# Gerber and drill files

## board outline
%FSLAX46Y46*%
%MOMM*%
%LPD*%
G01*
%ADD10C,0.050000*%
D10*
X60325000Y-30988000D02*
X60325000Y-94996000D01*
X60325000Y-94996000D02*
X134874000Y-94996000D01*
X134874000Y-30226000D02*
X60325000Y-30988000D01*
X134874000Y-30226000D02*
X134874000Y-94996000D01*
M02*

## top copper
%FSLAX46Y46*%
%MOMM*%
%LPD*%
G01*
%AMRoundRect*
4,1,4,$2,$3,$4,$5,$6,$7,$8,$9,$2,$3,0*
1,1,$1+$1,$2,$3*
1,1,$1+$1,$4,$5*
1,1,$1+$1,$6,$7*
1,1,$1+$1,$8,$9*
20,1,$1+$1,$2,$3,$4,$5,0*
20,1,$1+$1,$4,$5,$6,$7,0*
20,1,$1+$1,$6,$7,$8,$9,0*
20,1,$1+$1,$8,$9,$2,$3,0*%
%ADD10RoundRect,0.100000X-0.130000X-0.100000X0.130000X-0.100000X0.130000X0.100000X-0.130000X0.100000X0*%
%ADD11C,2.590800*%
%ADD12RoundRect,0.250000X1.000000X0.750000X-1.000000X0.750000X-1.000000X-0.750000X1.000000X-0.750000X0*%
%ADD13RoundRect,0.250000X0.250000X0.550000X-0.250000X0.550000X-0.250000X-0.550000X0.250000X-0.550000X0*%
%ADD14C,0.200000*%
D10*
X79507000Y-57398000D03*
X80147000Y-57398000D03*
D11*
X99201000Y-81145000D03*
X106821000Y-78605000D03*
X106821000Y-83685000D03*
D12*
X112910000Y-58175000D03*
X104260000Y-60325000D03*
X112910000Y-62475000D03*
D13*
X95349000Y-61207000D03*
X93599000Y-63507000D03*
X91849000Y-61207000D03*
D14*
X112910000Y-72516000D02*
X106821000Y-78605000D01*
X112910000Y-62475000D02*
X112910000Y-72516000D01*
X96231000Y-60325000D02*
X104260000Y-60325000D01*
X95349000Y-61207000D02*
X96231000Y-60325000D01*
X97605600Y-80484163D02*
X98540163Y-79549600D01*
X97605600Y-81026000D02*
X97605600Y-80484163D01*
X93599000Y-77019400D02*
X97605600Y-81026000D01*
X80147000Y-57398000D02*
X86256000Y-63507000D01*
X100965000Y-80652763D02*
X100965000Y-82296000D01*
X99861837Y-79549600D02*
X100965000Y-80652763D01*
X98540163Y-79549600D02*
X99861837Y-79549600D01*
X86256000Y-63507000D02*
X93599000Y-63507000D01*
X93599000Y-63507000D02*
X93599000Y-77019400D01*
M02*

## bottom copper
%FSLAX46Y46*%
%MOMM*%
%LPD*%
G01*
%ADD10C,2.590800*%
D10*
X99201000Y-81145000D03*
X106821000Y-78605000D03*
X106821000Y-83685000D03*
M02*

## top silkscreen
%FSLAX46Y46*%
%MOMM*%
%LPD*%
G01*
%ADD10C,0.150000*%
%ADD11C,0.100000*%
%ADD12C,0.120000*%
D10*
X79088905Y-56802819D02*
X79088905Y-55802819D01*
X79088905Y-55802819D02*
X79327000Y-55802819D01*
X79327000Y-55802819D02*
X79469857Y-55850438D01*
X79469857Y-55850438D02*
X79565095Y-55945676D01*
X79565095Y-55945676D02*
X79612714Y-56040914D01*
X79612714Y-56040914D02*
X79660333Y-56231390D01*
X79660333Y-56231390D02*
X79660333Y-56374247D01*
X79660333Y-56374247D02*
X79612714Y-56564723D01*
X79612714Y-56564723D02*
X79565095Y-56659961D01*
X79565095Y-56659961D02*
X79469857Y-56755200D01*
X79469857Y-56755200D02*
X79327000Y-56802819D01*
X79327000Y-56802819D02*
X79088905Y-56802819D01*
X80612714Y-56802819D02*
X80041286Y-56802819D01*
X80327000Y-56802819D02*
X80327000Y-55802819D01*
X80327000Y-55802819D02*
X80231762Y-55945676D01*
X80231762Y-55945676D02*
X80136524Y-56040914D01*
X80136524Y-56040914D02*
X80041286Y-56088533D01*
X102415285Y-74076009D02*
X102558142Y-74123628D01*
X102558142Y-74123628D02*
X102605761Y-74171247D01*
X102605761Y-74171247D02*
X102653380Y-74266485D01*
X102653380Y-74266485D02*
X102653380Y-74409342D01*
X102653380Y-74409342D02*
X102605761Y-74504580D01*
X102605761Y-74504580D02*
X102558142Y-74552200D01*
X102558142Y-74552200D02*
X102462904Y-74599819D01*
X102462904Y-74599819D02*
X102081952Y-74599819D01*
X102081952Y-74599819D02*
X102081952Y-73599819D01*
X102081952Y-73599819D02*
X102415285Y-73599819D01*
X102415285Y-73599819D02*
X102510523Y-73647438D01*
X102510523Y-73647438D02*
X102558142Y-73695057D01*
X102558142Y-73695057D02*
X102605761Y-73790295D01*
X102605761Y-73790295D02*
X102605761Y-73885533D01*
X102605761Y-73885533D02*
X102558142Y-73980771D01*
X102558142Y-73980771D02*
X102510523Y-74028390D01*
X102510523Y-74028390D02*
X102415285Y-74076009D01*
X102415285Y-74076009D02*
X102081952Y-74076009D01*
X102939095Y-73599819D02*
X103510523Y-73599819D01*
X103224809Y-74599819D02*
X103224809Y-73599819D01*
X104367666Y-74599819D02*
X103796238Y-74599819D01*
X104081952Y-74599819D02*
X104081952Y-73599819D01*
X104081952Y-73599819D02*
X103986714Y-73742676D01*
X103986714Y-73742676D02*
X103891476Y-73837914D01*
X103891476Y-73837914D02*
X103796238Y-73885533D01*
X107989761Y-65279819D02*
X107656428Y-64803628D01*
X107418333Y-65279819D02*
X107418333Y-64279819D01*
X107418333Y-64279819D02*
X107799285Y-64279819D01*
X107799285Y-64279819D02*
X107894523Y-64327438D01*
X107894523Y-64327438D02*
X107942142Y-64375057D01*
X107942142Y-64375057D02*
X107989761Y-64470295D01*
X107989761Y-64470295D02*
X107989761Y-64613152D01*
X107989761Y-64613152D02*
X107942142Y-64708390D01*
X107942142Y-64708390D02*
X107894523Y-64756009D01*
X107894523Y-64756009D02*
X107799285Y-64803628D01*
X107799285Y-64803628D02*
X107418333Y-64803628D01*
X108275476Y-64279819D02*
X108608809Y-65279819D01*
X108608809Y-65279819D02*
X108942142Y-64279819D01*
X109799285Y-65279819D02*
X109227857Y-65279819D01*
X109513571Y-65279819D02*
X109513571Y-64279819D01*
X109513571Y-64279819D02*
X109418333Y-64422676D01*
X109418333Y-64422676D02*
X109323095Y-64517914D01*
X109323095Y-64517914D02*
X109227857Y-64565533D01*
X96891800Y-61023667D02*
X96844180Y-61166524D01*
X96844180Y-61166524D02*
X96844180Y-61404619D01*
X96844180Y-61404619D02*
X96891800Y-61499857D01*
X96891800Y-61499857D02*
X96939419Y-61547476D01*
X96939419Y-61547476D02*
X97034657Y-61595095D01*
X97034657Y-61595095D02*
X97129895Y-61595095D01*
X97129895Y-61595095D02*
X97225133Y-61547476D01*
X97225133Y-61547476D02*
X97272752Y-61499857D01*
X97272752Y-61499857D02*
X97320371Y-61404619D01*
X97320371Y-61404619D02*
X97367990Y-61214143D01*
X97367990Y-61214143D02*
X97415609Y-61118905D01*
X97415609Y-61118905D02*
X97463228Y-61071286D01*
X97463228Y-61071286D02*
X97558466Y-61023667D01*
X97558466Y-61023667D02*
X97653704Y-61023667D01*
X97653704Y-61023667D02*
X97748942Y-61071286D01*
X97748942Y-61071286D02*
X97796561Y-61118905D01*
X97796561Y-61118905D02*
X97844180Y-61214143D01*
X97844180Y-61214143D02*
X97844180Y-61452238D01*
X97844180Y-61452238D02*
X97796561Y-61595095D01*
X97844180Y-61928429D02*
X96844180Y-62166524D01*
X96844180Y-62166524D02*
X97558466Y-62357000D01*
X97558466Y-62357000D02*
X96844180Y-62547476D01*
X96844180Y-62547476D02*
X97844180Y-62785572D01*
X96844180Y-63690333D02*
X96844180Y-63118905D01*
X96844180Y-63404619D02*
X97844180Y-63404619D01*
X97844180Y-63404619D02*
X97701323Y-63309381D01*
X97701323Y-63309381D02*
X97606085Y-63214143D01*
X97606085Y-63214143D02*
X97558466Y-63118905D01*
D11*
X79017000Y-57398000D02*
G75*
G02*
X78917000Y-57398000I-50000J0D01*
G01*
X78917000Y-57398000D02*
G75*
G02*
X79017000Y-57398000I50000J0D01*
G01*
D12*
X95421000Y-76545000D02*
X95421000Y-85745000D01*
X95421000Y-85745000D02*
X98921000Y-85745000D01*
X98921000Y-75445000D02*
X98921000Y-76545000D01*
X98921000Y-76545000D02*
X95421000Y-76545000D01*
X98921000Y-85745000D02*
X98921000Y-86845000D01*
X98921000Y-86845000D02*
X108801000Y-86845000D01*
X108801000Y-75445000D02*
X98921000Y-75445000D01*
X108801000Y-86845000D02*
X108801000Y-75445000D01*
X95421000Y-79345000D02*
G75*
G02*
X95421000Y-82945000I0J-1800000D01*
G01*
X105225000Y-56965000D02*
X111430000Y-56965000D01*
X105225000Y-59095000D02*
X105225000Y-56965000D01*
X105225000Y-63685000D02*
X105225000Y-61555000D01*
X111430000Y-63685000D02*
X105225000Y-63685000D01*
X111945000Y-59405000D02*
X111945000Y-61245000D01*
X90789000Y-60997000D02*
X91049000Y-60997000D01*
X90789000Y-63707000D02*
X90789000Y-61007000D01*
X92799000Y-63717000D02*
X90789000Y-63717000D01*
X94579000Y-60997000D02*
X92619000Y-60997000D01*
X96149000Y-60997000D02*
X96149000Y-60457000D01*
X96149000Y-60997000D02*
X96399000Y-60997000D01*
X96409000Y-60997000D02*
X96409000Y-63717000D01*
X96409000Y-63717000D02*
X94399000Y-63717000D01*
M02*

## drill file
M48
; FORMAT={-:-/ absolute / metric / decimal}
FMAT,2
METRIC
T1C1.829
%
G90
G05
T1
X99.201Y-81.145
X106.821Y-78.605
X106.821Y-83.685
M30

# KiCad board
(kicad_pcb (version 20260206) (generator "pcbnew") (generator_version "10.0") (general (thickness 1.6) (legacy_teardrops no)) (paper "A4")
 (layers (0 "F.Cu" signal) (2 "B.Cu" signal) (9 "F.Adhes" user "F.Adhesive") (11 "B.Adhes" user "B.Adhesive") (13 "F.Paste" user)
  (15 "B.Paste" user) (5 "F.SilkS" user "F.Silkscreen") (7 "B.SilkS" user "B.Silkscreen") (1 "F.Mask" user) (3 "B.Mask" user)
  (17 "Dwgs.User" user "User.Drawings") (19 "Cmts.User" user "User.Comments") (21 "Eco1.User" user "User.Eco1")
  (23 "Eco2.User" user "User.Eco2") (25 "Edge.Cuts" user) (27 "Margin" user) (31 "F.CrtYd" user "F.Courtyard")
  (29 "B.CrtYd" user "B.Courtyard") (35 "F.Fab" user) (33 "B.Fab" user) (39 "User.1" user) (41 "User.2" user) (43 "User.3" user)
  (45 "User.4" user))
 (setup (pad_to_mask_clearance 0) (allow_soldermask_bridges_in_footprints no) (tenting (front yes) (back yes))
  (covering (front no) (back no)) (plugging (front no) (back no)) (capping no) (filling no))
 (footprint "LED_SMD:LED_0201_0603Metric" (layer "F.Cu") (at 79.827 57.398)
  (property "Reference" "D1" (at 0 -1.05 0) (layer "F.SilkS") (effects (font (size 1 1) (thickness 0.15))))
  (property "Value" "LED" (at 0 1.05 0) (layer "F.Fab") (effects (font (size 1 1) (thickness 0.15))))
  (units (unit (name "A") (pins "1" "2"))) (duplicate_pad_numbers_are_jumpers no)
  (fp_circle (center -0.86 0) (end -0.81 0) (stroke (width 0.1) (type solid)) (fill no) (layer "F.SilkS"))
  (pad "" smd roundrect (at -0.345 0) (size 0.318 0.36) (layers "F.Paste") (roundrect_rratio 0.25))
  (pad "" smd roundrect (at 0.345 0) (size 0.318 0.36) (layers "F.Paste") (roundrect_rratio 0.25))
  (pad "1" smd roundrect (at -0.32 0) (size 0.46 0.4) (layers "F.Cu" "F.Mask") (roundrect_rratio 0.25) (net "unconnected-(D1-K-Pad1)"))
  (pad "2" smd roundrect (at 0.32 0) (size 0.46 0.4) (layers "F.Cu" "F.Mask") (roundrect_rratio 0.25) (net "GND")))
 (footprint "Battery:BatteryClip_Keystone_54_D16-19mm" (layer "F.Cu") (at 99.201 81.145)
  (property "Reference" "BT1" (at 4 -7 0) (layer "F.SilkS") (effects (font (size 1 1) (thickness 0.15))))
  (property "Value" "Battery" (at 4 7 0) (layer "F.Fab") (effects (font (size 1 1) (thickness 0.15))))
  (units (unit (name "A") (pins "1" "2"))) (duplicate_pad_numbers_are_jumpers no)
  (fp_line (start -3.78 -4.6) (end -3.78 4.6) (stroke (width 0.12) (type default)) (layer "F.SilkS"))
  (fp_line (start -3.78 4.6) (end -0.28 4.6) (stroke (width 0.12) (type default)) (layer "F.SilkS"))
  (fp_line (start -0.28 -5.7) (end -0.28 -4.6) (stroke (width 0.12) (type default)) (layer "F.SilkS"))
  (fp_line (start -0.28 -4.6) (end -3.78 -4.6) (stroke (width 0.12) (type default)) (layer "F.SilkS"))
  (fp_line (start -0.28 4.6) (end -0.28 5.7) (stroke (width 0.12) (type default)) (layer "F.SilkS"))
  (fp_line (start -0.28 5.7) (end 9.6 5.7) (stroke (width 0.12) (type default)) (layer "F.SilkS"))
  (fp_line (start 9.6 -5.7) (end -0.28 -5.7) (stroke (width 0.12) (type default)) (layer "F.SilkS"))
  (fp_line (start 9.6 5.7) (end 9.6 -5.7) (stroke (width 0.12) (type default)) (layer "F.SilkS"))
  (fp_arc (start -3.78 -1.8) (mid -1.98 0) (end -3.78 1.8) (stroke (width 0.12) (type default)) (layer "F.SilkS"))
  (pad "1" thru_hole circle (at 0 0 180) (size 2.5908 2.5908) (drill 1.8288) (layers "*.Cu" "*.Mask") (remove_unused_layers no) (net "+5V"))
  (pad "1" thru_hole circle (at 7.62 -2.54 180) (size 2.5908 2.5908) (drill 1.8288) (layers "*.Cu" "*.Mask") (remove_unused_layers no)
   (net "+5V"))
  (pad "1" thru_hole circle (at 7.62 2.54 180) (size 2.5908 2.5908) (drill 1.8288) (layers "*.Cu" "*.Mask") (remove_unused_layers no)
   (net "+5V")))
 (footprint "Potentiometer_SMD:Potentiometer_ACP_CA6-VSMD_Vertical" (layer "F.Cu") (at 108.585 60.325 180)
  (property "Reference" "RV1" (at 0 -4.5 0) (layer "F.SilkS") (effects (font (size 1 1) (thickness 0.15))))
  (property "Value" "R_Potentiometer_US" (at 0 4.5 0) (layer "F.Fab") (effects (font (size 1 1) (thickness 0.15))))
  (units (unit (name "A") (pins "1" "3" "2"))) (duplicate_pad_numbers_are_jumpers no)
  (fp_line (start 3.36 3.36) (end -2.845 3.36) (stroke (width 0.12) (type solid)) (layer "F.SilkS"))
  (fp_line (start 3.36 1.23) (end 3.36 3.36) (stroke (width 0.12) (type solid)) (layer "F.SilkS"))
  (fp_line (start 3.36 -3.36) (end 3.36 -1.23) (stroke (width 0.12) (type solid)) (layer "F.SilkS"))
  (fp_line (start -2.845 -3.36) (end 3.36 -3.36) (stroke (width 0.12) (type solid)) (layer "F.SilkS"))
  (fp_line (start -3.36 0.92) (end -3.36 -0.92) (stroke (width 0.12) (type solid)) (layer "F.SilkS"))
  (pad "1" smd roundrect (at -4.325 2.15 180) (size 2.5 2) (layers "F.Cu" "F.Mask" "F.Paste") (roundrect_rratio 0.125)
   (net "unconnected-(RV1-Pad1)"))
  (pad "2" smd roundrect (at 4.325 0 180) (size 2.5 2) (layers "F.Cu" "F.Mask" "F.Paste") (roundrect_rratio 0.125) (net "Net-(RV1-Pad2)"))
  (pad "3" smd roundrect (at -4.325 -2.15 180) (size 2.5 2) (layers "F.Cu" "F.Mask" "F.Paste") (roundrect_rratio 0.125) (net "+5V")))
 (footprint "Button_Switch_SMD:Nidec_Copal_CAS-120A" (layer "F.Cu") (at 93.599 62.357 -90)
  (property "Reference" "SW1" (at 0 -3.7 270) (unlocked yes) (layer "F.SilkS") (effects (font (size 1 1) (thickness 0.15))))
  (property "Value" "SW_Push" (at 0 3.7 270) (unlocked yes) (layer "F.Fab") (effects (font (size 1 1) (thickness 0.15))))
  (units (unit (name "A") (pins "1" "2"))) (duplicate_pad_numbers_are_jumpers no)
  (fp_line (start -1.36 2.81) (end -1.36 2.55) (stroke (width 0.12) (type solid)) (layer "F.SilkS"))
  (fp_line (start 1.35 2.81) (end -1.35 2.81) (stroke (width 0.12) (type solid)) (layer "F.SilkS"))
  (fp_line (start 1.36 0.8) (end 1.36 2.81) (stroke (width 0.12) (type solid)) (layer "F.SilkS"))
  (fp_line (start -1.36 -0.98) (end -1.36 0.98) (stroke (width 0.12) (type solid)) (layer "F.SilkS"))
  (fp_line (start -1.36 -2.55) (end -1.9 -2.55) (stroke (width 0.12) (type default)) (layer "F.SilkS"))
  (fp_line (start -1.36 -2.55) (end -1.36 -2.8) (stroke (width 0.12) (type solid)) (layer "F.SilkS"))
  (fp_line (start -1.36 -2.81) (end 1.36 -2.81) (stroke (width 0.12) (type solid)) (layer "F.SilkS"))
  (fp_line (start 1.36 -2.81) (end 1.36 -0.8) (stroke (width 0.12) (type solid)) (layer "F.SilkS"))
  (pad "1" smd roundrect (at -1.15 -1.75 180) (size 1 1.6) (layers "F.Cu" "F.Mask" "F.Paste") (roundrect_rratio 0.25) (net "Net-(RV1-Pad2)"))
  (pad "2" smd roundrect (at 1.15 0 180) (size 1 1.6) (layers "F.Cu" "F.Mask" "F.Paste") (roundrect_rratio 0.25) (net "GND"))
  (pad "3" smd roundrect (at -1.15 1.75 180) (size 1 1.6) (layers "F.Cu" "F.Mask" "F.Paste") (roundrect_rratio 0.25)))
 (gr_line (start 60.325 30.988) (end 60.325 94.996) (stroke (width 0.05) (type default)) (layer "Edge.Cuts"))
 (gr_line (start 60.325 94.996) (end 134.874 94.996) (stroke (width 0.05) (type default)) (layer "Edge.Cuts"))
 (gr_line (start 134.874 30.226) (end 60.325 30.988) (stroke (width 0.05) (type default)) (layer "Edge.Cuts"))
 (gr_line (start 134.874 30.226) (end 134.874 94.996) (stroke (width 0.05) (type default)) (layer "Edge.Cuts"))
 (segment (start 112.91 72.516) (end 106.821 78.605) (width 0.2) (layer "F.Cu") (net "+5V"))
 (segment (start 112.91 62.475) (end 112.91 72.516) (width 0.2) (layer "F.Cu") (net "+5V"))
 (segment (start 96.231 60.325) (end 104.26 60.325) (width 0.2) (layer "F.Cu") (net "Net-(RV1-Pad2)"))
 (segment (start 95.349 61.207) (end 96.231 60.325) (width 0.2) (layer "F.Cu") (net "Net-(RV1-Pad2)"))
 (segment (start 97.6056 80.484163) (end 98.540163 79.5496) (width 0.2) (layer "F.Cu") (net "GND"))
 (segment (start 97.6056 81.026) (end 97.6056 80.484163) (width 0.2) (layer "F.Cu") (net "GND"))
 (segment (start 93.599 77.0194) (end 97.6056 81.026) (width 0.2) (layer "F.Cu") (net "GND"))
 (segment (start 80.147 57.398) (end 86.256 63.507) (width 0.2) (layer "F.Cu") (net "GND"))
 (segment (start 100.965 80.652763) (end 100.965 82.296) (width 0.2) (layer "F.Cu") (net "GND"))
 (segment (start 99.861837 79.5496) (end 100.965 80.652763) (width 0.2) (layer "F.Cu") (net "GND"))
 (segment (start 98.540163 79.5496) (end 99.861837 79.5496) (width 0.2) (layer "F.Cu") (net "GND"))
 (segment (start 86.256 63.507) (end 93.599 63.507) (width 0.2) (layer "F.Cu") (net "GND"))
 (segment (start 93.599 63.507) (end 93.599 77.0194) (width 0.2) (layer "F.Cu") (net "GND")))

